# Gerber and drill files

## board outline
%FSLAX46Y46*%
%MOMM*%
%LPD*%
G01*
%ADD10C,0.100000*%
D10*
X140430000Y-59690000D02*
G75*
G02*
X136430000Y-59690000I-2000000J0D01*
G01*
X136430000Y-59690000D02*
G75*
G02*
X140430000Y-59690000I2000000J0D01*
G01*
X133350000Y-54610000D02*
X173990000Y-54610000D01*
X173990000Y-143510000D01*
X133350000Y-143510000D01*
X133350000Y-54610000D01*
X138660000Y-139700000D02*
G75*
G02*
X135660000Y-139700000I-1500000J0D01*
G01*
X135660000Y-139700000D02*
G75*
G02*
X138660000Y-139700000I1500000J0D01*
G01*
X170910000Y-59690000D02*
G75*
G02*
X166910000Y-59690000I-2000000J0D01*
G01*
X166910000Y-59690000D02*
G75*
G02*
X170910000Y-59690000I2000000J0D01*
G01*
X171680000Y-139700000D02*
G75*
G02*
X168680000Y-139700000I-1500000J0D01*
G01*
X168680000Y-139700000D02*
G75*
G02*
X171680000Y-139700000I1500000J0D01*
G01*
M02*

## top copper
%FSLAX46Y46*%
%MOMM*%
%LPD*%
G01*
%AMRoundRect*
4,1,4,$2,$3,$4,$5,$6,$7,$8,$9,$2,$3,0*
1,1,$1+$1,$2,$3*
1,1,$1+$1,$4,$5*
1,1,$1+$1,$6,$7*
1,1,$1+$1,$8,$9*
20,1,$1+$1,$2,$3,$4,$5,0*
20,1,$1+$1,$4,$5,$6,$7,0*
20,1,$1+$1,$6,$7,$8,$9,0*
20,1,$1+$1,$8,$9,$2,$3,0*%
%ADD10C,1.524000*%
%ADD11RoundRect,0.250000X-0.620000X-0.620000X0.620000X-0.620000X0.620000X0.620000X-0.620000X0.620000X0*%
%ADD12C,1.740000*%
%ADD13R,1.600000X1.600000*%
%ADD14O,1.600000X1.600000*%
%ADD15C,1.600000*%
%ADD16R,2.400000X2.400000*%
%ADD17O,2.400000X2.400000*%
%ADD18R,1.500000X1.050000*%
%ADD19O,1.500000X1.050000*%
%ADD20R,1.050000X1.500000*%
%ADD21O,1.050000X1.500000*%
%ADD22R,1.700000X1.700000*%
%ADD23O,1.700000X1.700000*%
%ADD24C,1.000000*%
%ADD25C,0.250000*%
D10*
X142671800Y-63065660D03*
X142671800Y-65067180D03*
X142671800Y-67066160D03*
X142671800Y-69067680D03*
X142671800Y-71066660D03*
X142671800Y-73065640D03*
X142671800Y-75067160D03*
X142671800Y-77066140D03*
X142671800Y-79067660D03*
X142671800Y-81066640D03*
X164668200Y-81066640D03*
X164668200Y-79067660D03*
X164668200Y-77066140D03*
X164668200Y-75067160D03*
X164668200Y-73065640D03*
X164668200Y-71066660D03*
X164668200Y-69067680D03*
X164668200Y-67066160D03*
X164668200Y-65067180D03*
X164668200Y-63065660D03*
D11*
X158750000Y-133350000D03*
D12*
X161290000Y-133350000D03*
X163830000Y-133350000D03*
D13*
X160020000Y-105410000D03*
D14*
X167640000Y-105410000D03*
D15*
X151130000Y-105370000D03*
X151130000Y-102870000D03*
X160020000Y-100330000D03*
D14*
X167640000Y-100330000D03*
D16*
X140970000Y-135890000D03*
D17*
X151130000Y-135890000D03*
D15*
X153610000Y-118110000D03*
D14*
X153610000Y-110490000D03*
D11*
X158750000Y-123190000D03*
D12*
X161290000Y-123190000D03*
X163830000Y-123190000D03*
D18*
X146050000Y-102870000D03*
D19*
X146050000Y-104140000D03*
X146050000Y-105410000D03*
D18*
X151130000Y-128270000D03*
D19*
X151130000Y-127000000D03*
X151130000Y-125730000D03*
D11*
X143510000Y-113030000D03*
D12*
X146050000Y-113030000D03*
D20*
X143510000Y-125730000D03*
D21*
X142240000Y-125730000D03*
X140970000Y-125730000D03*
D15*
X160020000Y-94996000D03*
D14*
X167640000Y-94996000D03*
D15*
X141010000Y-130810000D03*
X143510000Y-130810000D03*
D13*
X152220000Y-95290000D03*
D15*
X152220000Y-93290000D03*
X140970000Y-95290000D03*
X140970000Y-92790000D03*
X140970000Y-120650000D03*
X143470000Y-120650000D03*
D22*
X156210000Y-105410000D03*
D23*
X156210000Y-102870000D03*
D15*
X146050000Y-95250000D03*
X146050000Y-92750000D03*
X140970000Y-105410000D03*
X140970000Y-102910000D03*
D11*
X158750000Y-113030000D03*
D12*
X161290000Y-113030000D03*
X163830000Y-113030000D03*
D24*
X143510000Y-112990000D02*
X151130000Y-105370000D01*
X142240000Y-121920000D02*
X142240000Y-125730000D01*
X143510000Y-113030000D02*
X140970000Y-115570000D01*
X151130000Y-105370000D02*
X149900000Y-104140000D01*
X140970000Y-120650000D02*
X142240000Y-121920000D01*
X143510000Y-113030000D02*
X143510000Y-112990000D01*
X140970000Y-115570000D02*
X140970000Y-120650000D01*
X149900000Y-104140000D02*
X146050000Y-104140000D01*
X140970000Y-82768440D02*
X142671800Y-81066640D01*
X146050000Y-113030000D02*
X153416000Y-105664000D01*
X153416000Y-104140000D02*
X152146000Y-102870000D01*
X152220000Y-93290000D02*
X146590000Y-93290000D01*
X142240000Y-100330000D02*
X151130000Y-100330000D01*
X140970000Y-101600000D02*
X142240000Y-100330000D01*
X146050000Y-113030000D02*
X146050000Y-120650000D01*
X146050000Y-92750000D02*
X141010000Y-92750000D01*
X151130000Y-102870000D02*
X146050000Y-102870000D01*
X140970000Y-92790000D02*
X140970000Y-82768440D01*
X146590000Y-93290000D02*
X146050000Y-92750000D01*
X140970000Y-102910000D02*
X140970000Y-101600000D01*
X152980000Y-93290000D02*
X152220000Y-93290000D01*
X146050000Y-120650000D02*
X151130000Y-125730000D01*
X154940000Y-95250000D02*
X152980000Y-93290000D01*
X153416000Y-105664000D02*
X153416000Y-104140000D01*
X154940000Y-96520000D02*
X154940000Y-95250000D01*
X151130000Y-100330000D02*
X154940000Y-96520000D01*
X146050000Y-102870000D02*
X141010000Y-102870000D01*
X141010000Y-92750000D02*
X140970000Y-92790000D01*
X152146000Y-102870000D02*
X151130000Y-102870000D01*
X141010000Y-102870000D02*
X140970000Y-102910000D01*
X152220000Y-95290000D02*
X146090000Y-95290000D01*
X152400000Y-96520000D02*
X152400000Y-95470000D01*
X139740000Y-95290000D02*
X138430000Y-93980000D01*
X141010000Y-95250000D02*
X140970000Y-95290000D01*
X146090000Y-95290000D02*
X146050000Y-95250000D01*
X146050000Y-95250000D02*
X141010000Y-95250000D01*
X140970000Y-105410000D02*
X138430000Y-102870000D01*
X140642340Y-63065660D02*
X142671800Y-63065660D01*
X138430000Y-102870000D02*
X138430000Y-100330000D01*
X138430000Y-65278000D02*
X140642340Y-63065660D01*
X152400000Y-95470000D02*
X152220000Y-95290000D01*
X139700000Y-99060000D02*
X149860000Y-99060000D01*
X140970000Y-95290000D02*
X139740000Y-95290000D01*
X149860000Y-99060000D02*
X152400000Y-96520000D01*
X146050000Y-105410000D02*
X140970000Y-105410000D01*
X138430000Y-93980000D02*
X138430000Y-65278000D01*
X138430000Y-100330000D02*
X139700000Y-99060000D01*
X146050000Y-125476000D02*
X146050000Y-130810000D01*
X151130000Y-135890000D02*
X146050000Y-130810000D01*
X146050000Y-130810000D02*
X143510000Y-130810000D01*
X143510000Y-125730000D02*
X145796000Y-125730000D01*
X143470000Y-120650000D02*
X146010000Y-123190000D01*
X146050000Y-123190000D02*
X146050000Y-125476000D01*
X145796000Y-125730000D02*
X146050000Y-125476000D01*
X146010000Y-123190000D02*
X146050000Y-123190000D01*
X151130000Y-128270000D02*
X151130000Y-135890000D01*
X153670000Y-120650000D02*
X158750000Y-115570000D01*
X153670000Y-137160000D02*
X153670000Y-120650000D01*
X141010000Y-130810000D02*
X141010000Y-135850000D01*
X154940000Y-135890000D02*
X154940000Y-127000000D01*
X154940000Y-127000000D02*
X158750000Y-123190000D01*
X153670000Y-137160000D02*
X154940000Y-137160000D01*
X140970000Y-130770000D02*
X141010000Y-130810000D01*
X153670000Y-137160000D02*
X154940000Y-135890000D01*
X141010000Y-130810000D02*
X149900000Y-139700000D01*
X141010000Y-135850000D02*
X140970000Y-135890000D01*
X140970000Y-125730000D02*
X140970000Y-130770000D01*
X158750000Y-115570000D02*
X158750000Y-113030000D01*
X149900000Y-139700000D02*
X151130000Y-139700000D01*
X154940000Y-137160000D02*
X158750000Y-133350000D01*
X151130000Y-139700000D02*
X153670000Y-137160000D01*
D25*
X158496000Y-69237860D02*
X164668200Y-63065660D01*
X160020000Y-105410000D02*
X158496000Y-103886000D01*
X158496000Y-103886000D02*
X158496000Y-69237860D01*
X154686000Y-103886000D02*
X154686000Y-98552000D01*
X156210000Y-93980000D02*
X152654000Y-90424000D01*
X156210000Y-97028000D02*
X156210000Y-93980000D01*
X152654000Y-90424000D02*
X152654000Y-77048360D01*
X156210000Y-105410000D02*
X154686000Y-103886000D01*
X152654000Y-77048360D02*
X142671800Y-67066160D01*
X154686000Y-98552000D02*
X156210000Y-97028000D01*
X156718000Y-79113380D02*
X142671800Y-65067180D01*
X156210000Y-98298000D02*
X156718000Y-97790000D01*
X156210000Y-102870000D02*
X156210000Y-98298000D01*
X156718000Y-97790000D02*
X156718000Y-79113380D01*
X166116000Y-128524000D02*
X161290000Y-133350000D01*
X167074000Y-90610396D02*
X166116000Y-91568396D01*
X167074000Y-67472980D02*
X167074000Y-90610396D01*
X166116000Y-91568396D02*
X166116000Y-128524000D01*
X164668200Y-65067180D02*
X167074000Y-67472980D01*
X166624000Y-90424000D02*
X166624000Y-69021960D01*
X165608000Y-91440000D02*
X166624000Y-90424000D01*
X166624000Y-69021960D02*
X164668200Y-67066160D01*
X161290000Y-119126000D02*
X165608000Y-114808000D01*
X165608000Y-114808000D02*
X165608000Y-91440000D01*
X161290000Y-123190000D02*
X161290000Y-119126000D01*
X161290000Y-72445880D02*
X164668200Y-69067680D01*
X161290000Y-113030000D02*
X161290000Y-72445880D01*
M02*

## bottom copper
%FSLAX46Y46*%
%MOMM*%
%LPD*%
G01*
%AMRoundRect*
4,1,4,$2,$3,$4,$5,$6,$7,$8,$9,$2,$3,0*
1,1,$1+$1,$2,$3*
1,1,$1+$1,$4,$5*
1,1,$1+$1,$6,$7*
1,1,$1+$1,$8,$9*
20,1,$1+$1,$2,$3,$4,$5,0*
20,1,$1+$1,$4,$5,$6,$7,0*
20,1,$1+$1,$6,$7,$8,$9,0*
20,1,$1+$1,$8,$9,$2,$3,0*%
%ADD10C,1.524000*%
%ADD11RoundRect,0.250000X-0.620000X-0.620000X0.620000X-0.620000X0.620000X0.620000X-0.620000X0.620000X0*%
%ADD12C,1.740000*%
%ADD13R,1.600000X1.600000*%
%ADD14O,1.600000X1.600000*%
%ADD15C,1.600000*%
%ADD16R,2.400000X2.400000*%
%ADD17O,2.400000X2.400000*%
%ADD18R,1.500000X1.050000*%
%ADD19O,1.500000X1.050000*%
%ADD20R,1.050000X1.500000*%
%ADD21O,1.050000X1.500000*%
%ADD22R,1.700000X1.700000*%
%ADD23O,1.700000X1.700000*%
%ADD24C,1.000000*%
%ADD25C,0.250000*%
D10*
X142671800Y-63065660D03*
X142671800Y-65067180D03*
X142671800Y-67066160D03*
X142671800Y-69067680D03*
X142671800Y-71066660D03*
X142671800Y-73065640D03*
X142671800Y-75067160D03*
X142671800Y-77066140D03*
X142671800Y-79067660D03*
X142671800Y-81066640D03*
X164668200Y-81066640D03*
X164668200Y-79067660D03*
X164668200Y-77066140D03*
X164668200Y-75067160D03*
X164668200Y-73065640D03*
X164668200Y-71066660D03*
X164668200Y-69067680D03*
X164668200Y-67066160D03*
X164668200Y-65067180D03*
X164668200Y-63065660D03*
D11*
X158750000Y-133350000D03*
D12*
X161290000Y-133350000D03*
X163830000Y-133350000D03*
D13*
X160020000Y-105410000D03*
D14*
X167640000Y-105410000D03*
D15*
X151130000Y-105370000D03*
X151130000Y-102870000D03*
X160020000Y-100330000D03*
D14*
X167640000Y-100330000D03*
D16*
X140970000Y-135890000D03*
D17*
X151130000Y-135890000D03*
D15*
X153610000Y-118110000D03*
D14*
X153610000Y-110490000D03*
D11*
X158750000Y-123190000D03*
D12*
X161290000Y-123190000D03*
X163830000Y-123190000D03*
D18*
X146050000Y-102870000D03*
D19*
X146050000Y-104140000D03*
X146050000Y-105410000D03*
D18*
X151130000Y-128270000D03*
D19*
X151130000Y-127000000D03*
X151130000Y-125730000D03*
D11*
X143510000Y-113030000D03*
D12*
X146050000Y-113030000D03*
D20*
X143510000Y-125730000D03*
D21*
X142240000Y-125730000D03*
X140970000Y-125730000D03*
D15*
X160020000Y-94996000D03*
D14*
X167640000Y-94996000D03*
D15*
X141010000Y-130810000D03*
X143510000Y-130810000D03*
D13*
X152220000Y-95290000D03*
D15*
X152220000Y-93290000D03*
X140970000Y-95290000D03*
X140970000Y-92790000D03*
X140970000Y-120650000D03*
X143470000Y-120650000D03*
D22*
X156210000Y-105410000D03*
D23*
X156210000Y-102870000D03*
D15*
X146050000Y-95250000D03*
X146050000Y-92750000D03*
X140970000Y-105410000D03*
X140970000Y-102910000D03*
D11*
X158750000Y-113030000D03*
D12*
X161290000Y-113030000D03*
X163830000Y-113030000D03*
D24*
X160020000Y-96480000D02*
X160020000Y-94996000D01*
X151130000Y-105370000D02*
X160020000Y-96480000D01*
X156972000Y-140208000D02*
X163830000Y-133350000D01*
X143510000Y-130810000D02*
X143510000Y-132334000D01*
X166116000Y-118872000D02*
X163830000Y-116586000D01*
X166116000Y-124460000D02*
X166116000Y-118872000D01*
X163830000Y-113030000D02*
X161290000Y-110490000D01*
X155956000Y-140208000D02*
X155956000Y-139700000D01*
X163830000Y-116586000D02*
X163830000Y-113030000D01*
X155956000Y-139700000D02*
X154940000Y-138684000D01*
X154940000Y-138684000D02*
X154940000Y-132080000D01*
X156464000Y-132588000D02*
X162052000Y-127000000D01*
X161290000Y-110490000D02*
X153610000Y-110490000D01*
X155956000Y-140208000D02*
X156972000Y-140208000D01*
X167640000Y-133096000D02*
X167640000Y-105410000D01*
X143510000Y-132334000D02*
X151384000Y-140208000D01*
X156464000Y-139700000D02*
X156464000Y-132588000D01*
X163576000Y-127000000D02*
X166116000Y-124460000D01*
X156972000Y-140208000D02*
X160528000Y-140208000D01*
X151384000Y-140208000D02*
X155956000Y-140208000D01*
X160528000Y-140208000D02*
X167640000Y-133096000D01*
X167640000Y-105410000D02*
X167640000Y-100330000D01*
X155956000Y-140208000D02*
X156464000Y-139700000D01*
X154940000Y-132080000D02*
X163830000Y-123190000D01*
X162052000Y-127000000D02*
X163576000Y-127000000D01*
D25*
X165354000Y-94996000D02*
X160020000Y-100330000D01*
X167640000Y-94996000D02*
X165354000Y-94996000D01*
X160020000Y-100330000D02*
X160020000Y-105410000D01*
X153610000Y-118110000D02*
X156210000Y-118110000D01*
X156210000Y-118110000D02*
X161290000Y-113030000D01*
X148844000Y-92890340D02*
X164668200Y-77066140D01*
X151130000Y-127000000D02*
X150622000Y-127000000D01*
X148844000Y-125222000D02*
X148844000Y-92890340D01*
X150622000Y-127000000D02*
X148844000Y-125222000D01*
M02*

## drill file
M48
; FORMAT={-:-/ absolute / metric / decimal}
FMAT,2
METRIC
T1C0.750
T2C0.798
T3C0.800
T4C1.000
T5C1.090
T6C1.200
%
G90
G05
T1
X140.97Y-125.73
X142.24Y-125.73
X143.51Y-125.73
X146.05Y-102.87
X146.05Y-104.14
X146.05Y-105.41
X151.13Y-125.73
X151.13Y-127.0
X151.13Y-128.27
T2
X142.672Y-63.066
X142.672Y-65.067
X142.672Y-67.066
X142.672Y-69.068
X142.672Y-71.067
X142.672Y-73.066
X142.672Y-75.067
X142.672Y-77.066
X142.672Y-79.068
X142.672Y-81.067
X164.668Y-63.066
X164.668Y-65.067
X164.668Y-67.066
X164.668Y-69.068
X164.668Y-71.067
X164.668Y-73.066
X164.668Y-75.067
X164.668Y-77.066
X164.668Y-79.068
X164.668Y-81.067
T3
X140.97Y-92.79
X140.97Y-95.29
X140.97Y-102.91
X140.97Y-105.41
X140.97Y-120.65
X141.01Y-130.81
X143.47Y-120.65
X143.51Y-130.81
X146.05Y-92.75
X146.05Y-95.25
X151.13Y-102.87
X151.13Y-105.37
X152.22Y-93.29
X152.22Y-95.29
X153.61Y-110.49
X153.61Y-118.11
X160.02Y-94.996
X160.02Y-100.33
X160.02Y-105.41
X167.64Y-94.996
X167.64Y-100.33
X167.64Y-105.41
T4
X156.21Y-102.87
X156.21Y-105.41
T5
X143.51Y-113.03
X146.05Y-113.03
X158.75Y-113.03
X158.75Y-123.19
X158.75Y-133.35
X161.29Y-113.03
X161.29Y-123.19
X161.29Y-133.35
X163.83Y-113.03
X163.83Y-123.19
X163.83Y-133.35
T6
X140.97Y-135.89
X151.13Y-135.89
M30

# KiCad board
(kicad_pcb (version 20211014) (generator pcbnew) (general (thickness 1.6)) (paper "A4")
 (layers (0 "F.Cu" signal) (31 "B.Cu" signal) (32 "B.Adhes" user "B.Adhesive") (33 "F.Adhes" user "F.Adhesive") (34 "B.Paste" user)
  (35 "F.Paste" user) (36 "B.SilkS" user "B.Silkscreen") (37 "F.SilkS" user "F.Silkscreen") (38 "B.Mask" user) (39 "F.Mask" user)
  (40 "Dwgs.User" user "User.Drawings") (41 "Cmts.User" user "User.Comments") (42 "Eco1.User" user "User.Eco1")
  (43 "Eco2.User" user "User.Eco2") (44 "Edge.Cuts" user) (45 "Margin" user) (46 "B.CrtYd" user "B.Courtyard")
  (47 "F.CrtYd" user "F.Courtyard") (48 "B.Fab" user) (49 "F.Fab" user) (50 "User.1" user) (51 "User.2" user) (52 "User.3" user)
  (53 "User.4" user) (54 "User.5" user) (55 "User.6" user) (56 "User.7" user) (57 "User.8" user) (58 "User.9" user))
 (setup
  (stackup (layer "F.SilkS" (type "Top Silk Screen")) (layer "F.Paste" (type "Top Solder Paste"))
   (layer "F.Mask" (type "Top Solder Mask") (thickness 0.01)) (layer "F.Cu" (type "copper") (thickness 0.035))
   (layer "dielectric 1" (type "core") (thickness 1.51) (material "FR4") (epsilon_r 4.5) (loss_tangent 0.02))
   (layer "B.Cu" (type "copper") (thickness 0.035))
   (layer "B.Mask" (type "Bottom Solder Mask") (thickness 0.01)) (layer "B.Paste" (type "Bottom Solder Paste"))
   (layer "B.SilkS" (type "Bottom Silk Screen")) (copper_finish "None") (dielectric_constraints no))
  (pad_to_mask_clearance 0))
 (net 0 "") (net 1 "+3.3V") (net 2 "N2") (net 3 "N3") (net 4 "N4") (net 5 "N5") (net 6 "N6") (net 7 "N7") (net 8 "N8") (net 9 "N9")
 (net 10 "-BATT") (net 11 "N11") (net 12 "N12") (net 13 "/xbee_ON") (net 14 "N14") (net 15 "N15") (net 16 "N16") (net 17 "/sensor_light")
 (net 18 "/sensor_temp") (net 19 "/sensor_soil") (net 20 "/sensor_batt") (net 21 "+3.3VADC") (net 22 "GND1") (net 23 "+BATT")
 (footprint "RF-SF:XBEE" (layer "F.Cu") (at 153.67 83.06562)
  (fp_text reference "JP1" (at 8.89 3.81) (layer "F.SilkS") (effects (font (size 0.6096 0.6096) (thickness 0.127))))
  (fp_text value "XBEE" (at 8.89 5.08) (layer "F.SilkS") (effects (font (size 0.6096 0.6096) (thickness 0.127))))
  (pad "1" thru_hole circle locked (at -10.9982 -19.99996) (size 1.524 1.524) (drill 0.79756) (layers *.Cu *.Mask) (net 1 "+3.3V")
   (solder_mask_margin 0.1016))
  (pad "2" thru_hole circle locked (at -10.9982 -17.99844) (size 1.524 1.524) (drill 0.79756) (layers *.Cu *.Mask) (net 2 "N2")
   (solder_mask_margin 0.1016))
  (pad "3" thru_hole circle locked (at -10.9982 -15.99946) (size 1.524 1.524) (drill 0.79756) (layers *.Cu *.Mask) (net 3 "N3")
   (solder_mask_margin 0.1016))
  (pad "4" thru_hole circle locked (at -10.9982 -13.99794) (size 1.524 1.524) (drill 0.79756) (layers *.Cu *.Mask) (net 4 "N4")
   (solder_mask_margin 0.1016))
  (pad "5" thru_hole circle locked (at -10.9982 -11.99896) (size 1.524 1.524) (drill 0.79756) (layers *.Cu *.Mask) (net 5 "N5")
   (solder_mask_margin 0.1016))
  (pad "6" thru_hole circle locked (at -10.9982 -9.99998) (size 1.524 1.524) (drill 0.79756) (layers *.Cu *.Mask) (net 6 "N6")
   (solder_mask_margin 0.1016))
  (pad "7" thru_hole circle locked (at -10.9982 -7.99846) (size 1.524 1.524) (drill 0.79756) (layers *.Cu *.Mask) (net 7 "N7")
   (solder_mask_margin 0.1016))
  (pad "8" thru_hole circle locked (at -10.9982 -5.99948) (size 1.524 1.524) (drill 0.79756) (layers *.Cu *.Mask) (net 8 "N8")
   (solder_mask_margin 0.1016))
  (pad "9" thru_hole circle locked (at -10.9982 -3.99796) (size 1.524 1.524) (drill 0.79756) (layers *.Cu *.Mask) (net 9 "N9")
   (solder_mask_margin 0.1016))
  (pad "10" thru_hole circle locked (at -10.9982 -1.99898) (size 1.524 1.524) (drill 0.79756) (layers *.Cu *.Mask) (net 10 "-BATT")
   (solder_mask_margin 0.1016))
  (pad "11" thru_hole circle locked (at 10.9982 -1.99898) (size 1.524 1.524) (drill 0.79756) (layers *.Cu *.Mask) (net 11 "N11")
   (solder_mask_margin 0.1016))
  (pad "12" thru_hole circle locked (at 10.9982 -3.99796) (size 1.524 1.524) (drill 0.79756) (layers *.Cu *.Mask) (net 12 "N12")
   (solder_mask_margin 0.1016))
  (pad "13" thru_hole circle locked (at 10.9982 -5.99948) (size 1.524 1.524) (drill 0.79756) (layers *.Cu *.Mask) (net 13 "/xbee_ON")
   (solder_mask_margin 0.1016))
  (pad "14" thru_hole circle locked (at 10.9982 -7.99846) (size 1.524 1.524) (drill 0.79756) (layers *.Cu *.Mask) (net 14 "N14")
   (solder_mask_margin 0.1016))
  (pad "15" thru_hole circle locked (at 10.9982 -9.99998) (size 1.524 1.524) (drill 0.79756) (layers *.Cu *.Mask) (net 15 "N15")
   (solder_mask_margin 0.1016))
  (pad "16" thru_hole circle locked (at 10.9982 -11.99896) (size 1.524 1.524) (drill 0.79756) (layers *.Cu *.Mask) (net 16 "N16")
   (solder_mask_margin 0.1016))
  (pad "17" thru_hole circle locked (at 10.9982 -13.99794) (size 1.524 1.524) (drill 0.79756) (layers *.Cu *.Mask) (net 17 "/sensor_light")
   (solder_mask_margin 0.1016))
  (pad "18" thru_hole circle locked (at 10.9982 -15.99946) (size 1.524 1.524) (drill 0.79756) (layers *.Cu *.Mask) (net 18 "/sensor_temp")
   (solder_mask_margin 0.1016))
  (pad "19" thru_hole circle locked (at 10.9982 -17.99844) (size 1.524 1.524) (drill 0.79756) (layers *.Cu *.Mask) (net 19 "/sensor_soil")
   (solder_mask_margin 0.1016))
  (pad "20" thru_hole circle locked (at 10.9982 -19.99996) (size 1.524 1.524) (drill 0.79756) (layers *.Cu *.Mask) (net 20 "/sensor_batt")
   (solder_mask_margin 0.1016)))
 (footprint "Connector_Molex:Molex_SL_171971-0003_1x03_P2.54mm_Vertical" (layer "F.Cu") (at 158.75 133.35)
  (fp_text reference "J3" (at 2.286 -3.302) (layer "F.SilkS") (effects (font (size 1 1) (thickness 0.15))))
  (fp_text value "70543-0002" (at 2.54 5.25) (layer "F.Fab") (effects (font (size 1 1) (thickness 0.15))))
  (pad "1" thru_hole roundrect (at 0 0) (size 1.74 1.74) (drill 1.09) (layers *.Cu *.Mask) (roundrect_rratio 0.1436781609)
   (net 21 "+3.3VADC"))
  (pad "2" thru_hole circle (at 2.54 0) (size 1.74 1.74) (drill 1.09) (layers *.Cu *.Mask) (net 19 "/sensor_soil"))
  (pad "3" thru_hole circle (at 5.08 0) (size 1.74 1.74) (drill 1.09) (layers *.Cu *.Mask) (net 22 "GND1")))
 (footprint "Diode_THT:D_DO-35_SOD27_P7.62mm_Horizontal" (layer "F.Cu") (at 160.02 105.41)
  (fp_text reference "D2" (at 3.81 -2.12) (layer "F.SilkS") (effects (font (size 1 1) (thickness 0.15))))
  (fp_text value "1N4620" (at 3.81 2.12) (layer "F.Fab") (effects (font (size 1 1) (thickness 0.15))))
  (pad "1" thru_hole rect (at 0 0) (size 1.6 1.6) (drill 0.8) (layers *.Cu *.Mask) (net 20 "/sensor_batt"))
  (pad "2" thru_hole oval (at 7.62 0) (size 1.6 1.6) (drill 0.8) (layers *.Cu *.Mask) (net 22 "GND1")))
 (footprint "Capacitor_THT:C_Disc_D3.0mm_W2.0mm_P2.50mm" (layer "F.Cu") (at 151.13 105.37 90)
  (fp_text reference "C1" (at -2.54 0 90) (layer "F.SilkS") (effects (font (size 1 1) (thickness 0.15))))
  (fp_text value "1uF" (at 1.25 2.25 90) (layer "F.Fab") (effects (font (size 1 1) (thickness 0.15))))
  (pad "1" thru_hole circle (at 0 0 90) (size 1.6 1.6) (drill 0.8) (layers *.Cu *.Mask) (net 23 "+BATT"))
  (pad "2" thru_hole circle (at 2.5 0 90) (size 1.6 1.6) (drill 0.8) (layers *.Cu *.Mask) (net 10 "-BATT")))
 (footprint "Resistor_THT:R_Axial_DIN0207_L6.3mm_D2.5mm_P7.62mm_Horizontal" (layer "F.Cu") (at 160.02 100.33)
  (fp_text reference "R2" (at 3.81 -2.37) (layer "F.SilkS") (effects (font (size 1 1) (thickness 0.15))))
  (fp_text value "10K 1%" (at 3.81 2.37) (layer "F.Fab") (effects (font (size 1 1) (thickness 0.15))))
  (pad "1" thru_hole circle (at 0 0) (size 1.6 1.6) (drill 0.8) (layers *.Cu *.Mask) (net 20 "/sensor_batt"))
  (pad "2" thru_hole oval (at 7.62 0) (size 1.6 1.6) (drill 0.8) (layers *.Cu *.Mask) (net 22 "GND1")))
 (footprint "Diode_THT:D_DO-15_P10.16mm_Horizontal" (layer "F.Cu") (at 140.97 135.89)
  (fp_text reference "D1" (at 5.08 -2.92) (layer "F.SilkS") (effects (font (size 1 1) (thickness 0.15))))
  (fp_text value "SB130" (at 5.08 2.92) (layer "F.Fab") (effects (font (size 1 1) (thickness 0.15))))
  (pad "1" thru_hole rect (at 0 0) (size 2.4 2.4) (drill 1.2) (layers *.Cu *.Mask) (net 21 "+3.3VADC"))
  (pad "2" thru_hole oval (at 10.16 0) (size 2.4 2.4) (drill 1.2) (layers *.Cu *.Mask) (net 22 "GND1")))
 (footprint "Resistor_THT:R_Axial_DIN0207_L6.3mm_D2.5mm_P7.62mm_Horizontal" (layer "F.Cu") (at 153.61 118.11 90)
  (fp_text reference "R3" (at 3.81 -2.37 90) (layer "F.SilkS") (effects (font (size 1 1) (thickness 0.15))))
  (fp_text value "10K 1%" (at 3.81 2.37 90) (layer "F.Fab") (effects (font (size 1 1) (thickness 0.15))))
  (pad "1" thru_hole circle (at 0 0 90) (size 1.6 1.6) (drill 0.8) (layers *.Cu *.Mask) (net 17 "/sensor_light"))
  (pad "2" thru_hole oval (at 7.62 0 90) (size 1.6 1.6) (drill 0.8) (layers *.Cu *.Mask) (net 22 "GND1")))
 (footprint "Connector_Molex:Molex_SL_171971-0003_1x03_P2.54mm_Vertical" (layer "F.Cu") (at 158.75 123.19)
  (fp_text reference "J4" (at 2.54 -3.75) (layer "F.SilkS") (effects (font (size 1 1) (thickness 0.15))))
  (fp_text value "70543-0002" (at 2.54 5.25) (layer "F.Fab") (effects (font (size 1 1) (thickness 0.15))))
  (pad "1" thru_hole roundrect (at 0 0) (size 1.74 1.74) (drill 1.09) (layers *.Cu *.Mask) (roundrect_rratio 0.1436781609)
   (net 21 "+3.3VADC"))
  (pad "2" thru_hole circle (at 2.54 0) (size 1.74 1.74) (drill 1.09) (layers *.Cu *.Mask) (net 18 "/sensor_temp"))
  (pad "3" thru_hole circle (at 5.08 0) (size 1.74 1.74) (drill 1.09) (layers *.Cu *.Mask) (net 22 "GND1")))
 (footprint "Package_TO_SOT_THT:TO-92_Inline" (layer "F.Cu") (at 146.05 102.87 -90)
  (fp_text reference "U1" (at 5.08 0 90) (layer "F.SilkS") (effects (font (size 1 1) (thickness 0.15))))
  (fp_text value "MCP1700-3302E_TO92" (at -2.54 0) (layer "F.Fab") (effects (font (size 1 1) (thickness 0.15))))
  (pad "1" thru_hole rect (at 0 0 270) (size 1.05 1.5) (drill 0.75) (layers *.Cu *.Mask) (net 10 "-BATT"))
  (pad "2" thru_hole oval (at 1.27 0 270) (size 1.05 1.5) (drill 0.75) (layers *.Cu *.Mask) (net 23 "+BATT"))
  (pad "3" thru_hole oval (at 2.54 0 270) (size 1.05 1.5) (drill 0.75) (layers *.Cu *.Mask) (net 1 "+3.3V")))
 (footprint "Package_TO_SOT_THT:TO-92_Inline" (layer "F.Cu") (at 151.13 128.27 90)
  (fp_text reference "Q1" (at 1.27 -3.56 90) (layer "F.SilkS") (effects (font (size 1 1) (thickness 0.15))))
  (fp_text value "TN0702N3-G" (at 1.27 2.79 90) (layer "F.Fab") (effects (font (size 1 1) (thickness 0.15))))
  (pad "1" thru_hole rect (at 0 0 90) (size 1.05 1.5) (drill 0.75) (layers *.Cu *.Mask) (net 22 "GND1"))
  (pad "2" thru_hole oval (at 1.27 0 90) (size 1.05 1.5) (drill 0.75) (layers *.Cu *.Mask) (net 13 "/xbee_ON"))
  (pad "3" thru_hole oval (at 2.54 0 90) (size 1.05 1.5) (drill 0.75) (layers *.Cu *.Mask) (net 10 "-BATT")))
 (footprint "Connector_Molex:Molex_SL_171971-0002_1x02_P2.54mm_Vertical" (layer "F.Cu") (at 143.51 113.03)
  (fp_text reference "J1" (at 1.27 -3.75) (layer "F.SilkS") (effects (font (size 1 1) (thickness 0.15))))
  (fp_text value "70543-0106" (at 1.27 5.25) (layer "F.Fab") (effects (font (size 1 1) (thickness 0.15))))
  (pad "1" thru_hole roundrect (at 0 0) (size 1.74 1.74) (drill 1.09) (layers *.Cu *.Mask) (roundrect_rratio 0.1436781609) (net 23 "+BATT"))
  (pad "2" thru_hole circle (at 2.54 0) (size 1.74 1.74) (drill 1.09) (layers *.Cu *.Mask) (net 10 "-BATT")))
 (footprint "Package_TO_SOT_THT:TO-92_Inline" (layer "F.Cu") (at 143.51 125.73 180)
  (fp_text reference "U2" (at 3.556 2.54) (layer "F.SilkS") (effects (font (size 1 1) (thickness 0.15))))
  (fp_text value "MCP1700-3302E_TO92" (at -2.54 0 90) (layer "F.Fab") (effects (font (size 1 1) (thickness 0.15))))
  (pad "1" thru_hole rect (at 0 0 180) (size 1.05 1.5) (drill 0.75) (layers *.Cu *.Mask) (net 22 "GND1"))
  (pad "2" thru_hole oval (at 1.27 0 180) (size 1.05 1.5) (drill 0.75) (layers *.Cu *.Mask) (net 23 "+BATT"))
  (pad "3" thru_hole oval (at 2.54 0 180) (size 1.05 1.5) (drill 0.75) (layers *.Cu *.Mask) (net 21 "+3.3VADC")))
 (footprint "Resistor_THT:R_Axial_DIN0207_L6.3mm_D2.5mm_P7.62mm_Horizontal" (layer "F.Cu") (at 160.02 94.996)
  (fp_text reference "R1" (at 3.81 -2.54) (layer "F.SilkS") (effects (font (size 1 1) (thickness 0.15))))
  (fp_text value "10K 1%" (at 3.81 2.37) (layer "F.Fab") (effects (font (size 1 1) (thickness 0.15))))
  (pad "1" thru_hole circle (at 0 0) (size 1.6 1.6) (drill 0.8) (layers *.Cu *.Mask) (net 23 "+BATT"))
  (pad "2" thru_hole oval (at 7.62 0) (size 1.6 1.6) (drill 0.8) (layers *.Cu *.Mask) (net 20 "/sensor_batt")))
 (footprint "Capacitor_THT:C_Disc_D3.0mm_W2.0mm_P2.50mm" (layer "F.Cu") (at 141.01 130.81)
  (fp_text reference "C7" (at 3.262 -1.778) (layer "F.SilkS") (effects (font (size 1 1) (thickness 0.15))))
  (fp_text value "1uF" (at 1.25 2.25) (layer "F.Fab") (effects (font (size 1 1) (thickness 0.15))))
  (pad "1" thru_hole circle (at 0 0) (size 1.6 1.6) (drill 0.8) (layers *.Cu *.Mask) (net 21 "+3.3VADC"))
  (pad "2" thru_hole circle (at 2.5 0) (size 1.6 1.6) (drill 0.8) (layers *.Cu *.Mask) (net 22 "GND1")))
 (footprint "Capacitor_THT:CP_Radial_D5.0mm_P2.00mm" (layer "F.Cu") (at 152.22 95.29 90)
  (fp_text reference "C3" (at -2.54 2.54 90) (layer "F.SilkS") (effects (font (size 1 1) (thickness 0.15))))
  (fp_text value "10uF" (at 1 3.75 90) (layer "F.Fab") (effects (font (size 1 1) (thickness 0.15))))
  (pad "1" thru_hole rect (at 0 0 90) (size 1.6 1.6) (drill 0.8) (layers *.Cu *.Mask) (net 1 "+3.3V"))
  (pad "2" thru_hole circle (at 2 0 90) (size 1.6 1.6) (drill 0.8) (layers *.Cu *.Mask) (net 10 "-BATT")))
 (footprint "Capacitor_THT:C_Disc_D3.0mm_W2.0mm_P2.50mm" (layer "F.Cu") (at 140.97 95.29 90)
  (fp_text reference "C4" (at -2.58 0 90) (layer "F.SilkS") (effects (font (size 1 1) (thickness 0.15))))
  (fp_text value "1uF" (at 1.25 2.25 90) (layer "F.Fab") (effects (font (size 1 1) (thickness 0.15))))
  (pad "1" thru_hole circle (at 0 0 90) (size 1.6 1.6) (drill 0.8) (layers *.Cu *.Mask) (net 1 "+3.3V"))
  (pad "2" thru_hole circle (at 2.5 0 90) (size 1.6 1.6) (drill 0.8) (layers *.Cu *.Mask) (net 10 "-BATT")))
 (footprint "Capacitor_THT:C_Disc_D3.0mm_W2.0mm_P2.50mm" (layer "F.Cu") (at 140.97 120.65)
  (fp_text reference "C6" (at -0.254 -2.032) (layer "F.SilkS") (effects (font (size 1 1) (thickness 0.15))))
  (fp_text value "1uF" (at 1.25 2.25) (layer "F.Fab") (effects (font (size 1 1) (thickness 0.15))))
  (pad "1" thru_hole circle (at 0 0) (size 1.6 1.6) (drill 0.8) (layers *.Cu *.Mask) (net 23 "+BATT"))
  (pad "2" thru_hole circle (at 2.5 0) (size 1.6 1.6) (drill 0.8) (layers *.Cu *.Mask) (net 22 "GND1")))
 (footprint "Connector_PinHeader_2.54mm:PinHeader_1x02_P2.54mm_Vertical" (layer "F.Cu") (at 156.21 105.41 180)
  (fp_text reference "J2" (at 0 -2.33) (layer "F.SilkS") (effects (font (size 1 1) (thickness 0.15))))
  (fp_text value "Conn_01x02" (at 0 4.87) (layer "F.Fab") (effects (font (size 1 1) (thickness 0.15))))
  (pad "1" thru_hole rect (at 0 0 180) (size 1.7 1.7) (drill 1) (layers *.Cu *.Mask) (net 3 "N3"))
  (pad "2" thru_hole oval (at 0 2.54 180) (size 1.7 1.7) (drill 1) (layers *.Cu *.Mask) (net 2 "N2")))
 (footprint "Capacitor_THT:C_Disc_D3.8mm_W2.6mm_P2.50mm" (layer "F.Cu") (at 146.05 95.25 90)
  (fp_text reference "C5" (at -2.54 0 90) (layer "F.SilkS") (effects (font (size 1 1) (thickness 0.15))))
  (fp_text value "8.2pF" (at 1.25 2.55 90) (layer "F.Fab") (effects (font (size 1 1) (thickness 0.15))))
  (pad "1" thru_hole circle (at 0 0 90) (size 1.6 1.6) (drill 0.8) (layers *.Cu *.Mask) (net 1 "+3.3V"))
  (pad "2" thru_hole circle (at 2.5 0 90) (size 1.6 1.6) (drill 0.8) (layers *.Cu *.Mask) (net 10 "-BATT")))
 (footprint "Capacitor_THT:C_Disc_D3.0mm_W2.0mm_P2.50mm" (layer "F.Cu") (at 140.97 105.41 90)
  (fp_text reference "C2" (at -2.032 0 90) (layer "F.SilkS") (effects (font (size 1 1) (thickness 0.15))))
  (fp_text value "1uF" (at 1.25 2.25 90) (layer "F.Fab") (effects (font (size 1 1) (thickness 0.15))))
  (pad "1" thru_hole circle (at 0 0 90) (size 1.6 1.6) (drill 0.8) (layers *.Cu *.Mask) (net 1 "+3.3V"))
  (pad "2" thru_hole circle (at 2.5 0 90) (size 1.6 1.6) (drill 0.8) (layers *.Cu *.Mask) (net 10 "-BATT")))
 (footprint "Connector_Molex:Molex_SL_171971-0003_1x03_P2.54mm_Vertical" (layer "F.Cu") (at 158.75 113.03)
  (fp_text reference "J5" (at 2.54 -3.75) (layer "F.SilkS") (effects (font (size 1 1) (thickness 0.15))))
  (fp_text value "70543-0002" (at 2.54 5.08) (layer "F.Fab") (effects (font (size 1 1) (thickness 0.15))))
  (pad "1" thru_hole roundrect (at 0 0) (size 1.74 1.74) (drill 1.09) (layers *.Cu *.Mask) (roundrect_rratio 0.1436781609)
   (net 21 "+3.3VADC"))
  (pad "2" thru_hole circle (at 2.54 0) (size 1.74 1.74) (drill 1.09) (layers *.Cu *.Mask) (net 17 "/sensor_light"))
  (pad "3" thru_hole circle (at 5.08 0) (size 1.74 1.74) (drill 1.09) (layers *.Cu *.Mask) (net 22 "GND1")))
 (gr_circle (center 138.43 59.69) (end 140.43 59.69) (layer "Edge.Cuts") (width 0.1) (fill none))
 (gr_rect (start 133.35 143.51) (end 173.99 54.61) (layer "Edge.Cuts") (width 0.1) (fill none))
 (gr_circle (center 137.16 139.7) (end 138.66 139.7) (layer "Edge.Cuts") (width 0.1) (fill none))
 (gr_circle (center 168.91 59.69) (end 170.91 59.69) (layer "Edge.Cuts") (width 0.1) (fill none))
 (gr_circle (center 170.18 139.7) (end 171.68 139.7) (layer "Edge.Cuts") (width 0.1) (fill none))
 (segment (start 143.51 112.99) (end 151.13 105.37) (width 1) (layer "F.Cu") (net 23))
 (segment (start 142.24 121.92) (end 142.24 125.73) (width 1) (layer "F.Cu") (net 23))
 (segment (start 143.51 113.03) (end 140.97 115.57) (width 1) (layer "F.Cu") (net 23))
 (segment (start 151.13 105.37) (end 149.9 104.14) (width 1) (layer "F.Cu") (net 23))
 (segment (start 140.97 120.65) (end 142.24 121.92) (width 1) (layer "F.Cu") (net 23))
 (segment (start 143.51 113.03) (end 143.51 112.99) (width 1) (layer "F.Cu") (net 23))
 (segment (start 140.97 115.57) (end 140.97 120.65) (width 1) (layer "F.Cu") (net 23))
 (segment (start 149.9 104.14) (end 146.05 104.14) (width 1) (layer "F.Cu") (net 23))
 (segment (start 160.02 96.48) (end 160.02 94.996) (width 1) (layer "B.Cu") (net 23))
 (segment (start 151.13 105.37) (end 160.02 96.48) (width 1) (layer "B.Cu") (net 23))
 (segment (start 140.97 82.76844) (end 142.6718 81.06664) (width 1) (layer "F.Cu") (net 10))
 (segment (start 146.05 113.03) (end 153.416 105.664) (width 1) (layer "F.Cu") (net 10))
 (segment (start 153.416 104.14) (end 152.146 102.87) (width 1) (layer "F.Cu") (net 10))
 (segment (start 152.22 93.29) (end 146.59 93.29) (width 1) (layer "F.Cu") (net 10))
 (segment (start 142.24 100.33) (end 151.13 100.33) (width 1) (layer "F.Cu") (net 10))
 (segment (start 140.97 101.6) (end 142.24 100.33) (width 1) (layer "F.Cu") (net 10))
 (segment (start 146.05 113.03) (end 146.05 120.65) (width 1) (layer "F.Cu") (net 10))
 (segment (start 146.05 92.75) (end 141.01 92.75) (width 1) (layer "F.Cu") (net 10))
 (segment (start 151.13 102.87) (end 146.05 102.87) (width 1) (layer "F.Cu") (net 10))
 (segment (start 140.97 92.79) (end 140.97 82.76844) (width 1) (layer "F.Cu") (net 10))
 (segment (start 146.59 93.29) (end 146.05 92.75) (width 1) (layer "F.Cu") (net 10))
 (segment (start 140.97 102.91) (end 140.97 101.6) (width 1) (layer "F.Cu") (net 10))
 (segment (start 152.98 93.29) (end 152.22 93.29) (width 1) (layer "F.Cu") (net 10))
 (segment (start 146.05 120.65) (end 151.13 125.73) (width 1) (layer "F.Cu") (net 10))
 (segment (start 154.94 95.25) (end 152.98 93.29) (width 1) (layer "F.Cu") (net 10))
 (segment (start 153.416 105.664) (end 153.416 104.14) (width 1) (layer "F.Cu") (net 10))
 (segment (start 154.94 96.52) (end 154.94 95.25) (width 1) (layer "F.Cu") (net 10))
 (segment (start 151.13 100.33) (end 154.94 96.52) (width 1) (layer "F.Cu") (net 10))
 (segment (start 146.05 102.87) (end 141.01 102.87) (width 1) (layer "F.Cu") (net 10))
 (segment (start 141.01 92.75) (end 140.97 92.79) (width 1) (layer "F.Cu") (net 10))
 (segment (start 152.146 102.87) (end 151.13 102.87) (width 1) (layer "F.Cu") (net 10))
 (segment (start 141.01 102.87) (end 140.97 102.91) (width 1) (layer "F.Cu") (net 10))
 (segment (start 152.22 95.29) (end 146.09 95.29) (width 1) (layer "F.Cu") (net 1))
 (segment (start 152.4 96.52) (end 152.4 95.47) (width 1) (layer "F.Cu") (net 1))
 (segment (start 139.74 95.29) (end 138.43 93.98) (width 1) (layer "F.Cu") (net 1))
 (segment (start 141.01 95.25) (end 140.97 95.29) (width 1) (layer "F.Cu") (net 1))
 (segment (start 146.09 95.29) (end 146.05 95.25) (width 1) (layer "F.Cu") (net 1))
 (segment (start 146.05 95.25) (end 141.01 95.25) (width 1) (layer "F.Cu") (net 1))
 (segment (start 140.97 105.41) (end 138.43 102.87) (width 1) (layer "F.Cu") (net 1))
 (segment (start 140.64234 63.06566) (end 142.6718 63.06566) (width 1) (layer "F.Cu") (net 1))
 (segment (start 138.43 102.87) (end 138.43 100.33) (width 1) (layer "F.Cu") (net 1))
 (segment (start 138.43 65.278) (end 140.64234 63.06566) (width 1) (layer "F.Cu") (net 1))
 (segment (start 152.4 95.47) (end 152.22 95.29) (width 1) (layer "F.Cu") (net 1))
 (segment (start 139.7 99.06) (end 149.86 99.06) (width 1) (layer "F.Cu") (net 1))
 (segment (start 140.97 95.29) (end 139.74 95.29) (width 1) (layer "F.Cu") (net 1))
 (segment (start 149.86 99.06) (end 152.4 96.52) (width 1) (layer "F.Cu") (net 1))
 (segment (start 146.05 105.41) (end 140.97 105.41) (width 1) (layer "F.Cu") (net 1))
 (segment (start 138.43 93.98) (end 138.43 65.278) (width 1) (layer "F.Cu") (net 1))
 (segment (start 138.43 100.33) (end 139.7 99.06) (width 1) (layer "F.Cu") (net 1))
 (segment (start 146.05 125.476) (end 146.05 130.81) (width 1) (layer "F.Cu") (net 22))
 (segment (start 151.13 135.89) (end 146.05 130.81) (width 1) (layer "F.Cu") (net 22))
 (segment (start 146.05 130.81) (end 143.51 130.81) (width 1) (layer "F.Cu") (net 22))
 (segment (start 143.51 125.73) (end 145.796 125.73) (width 1) (layer "F.Cu") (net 22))
 (segment (start 143.47 120.65) (end 146.01 123.19) (width 1) (layer "F.Cu") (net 22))
 (segment (start 146.05 123.19) (end 146.05 125.476) (width 1) (layer "F.Cu") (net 22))
 (segment (start 145.796 125.73) (end 146.05 125.476) (width 1) (layer "F.Cu") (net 22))
 (segment (start 146.01 123.19) (end 146.05 123.19) (width 1) (layer "F.Cu") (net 22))
 (segment (start 151.13 128.27) (end 151.13 135.89) (width 1) (layer "F.Cu") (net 22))
 (segment (start 156.972 140.208) (end 163.83 133.35) (width 1) (layer "B.Cu") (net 22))
 (segment (start 143.51 130.81) (end 143.51 132.334) (width 1) (layer "B.Cu") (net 22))
 (segment (start 166.116 118.872) (end 163.83 116.586) (width 1) (layer "B.Cu") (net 22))
 (segment (start 166.116 124.46) (end 166.116 118.872) (width 1) (layer "B.Cu") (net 22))
 (segment (start 163.83 113.03) (end 161.29 110.49) (width 1) (layer "B.Cu") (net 22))
 (segment (start 155.956 140.208) (end 155.956 139.7) (width 1) (layer "B.Cu") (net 22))
 (segment (start 163.83 116.586) (end 163.83 113.03) (width 1) (layer "B.Cu") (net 22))
 (segment (start 155.956 139.7) (end 154.94 138.684) (width 1) (layer "B.Cu") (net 22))
 (segment (start 154.94 138.684) (end 154.94 132.08) (width 1) (layer "B.Cu") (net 22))
 (segment (start 156.464 132.588) (end 162.052 127) (width 1) (layer "B.Cu") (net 22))
 (segment (start 161.29 110.49) (end 153.61 110.49) (width 1) (layer "B.Cu") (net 22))
 (segment (start 155.956 140.208) (end 156.972 140.208) (width 1) (layer "B.Cu") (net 22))
 (segment (start 167.64 133.096) (end 167.64 105.41) (width 1) (layer "B.Cu") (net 22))
 (segment (start 143.51 132.334) (end 151.384 140.208) (width 1) (layer "B.Cu") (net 22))
 (segment (start 156.464 139.7) (end 156.464 132.588) (width 1) (layer "B.Cu") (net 22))
 (segment (start 163.576 127) (end 166.116 124.46) (width 1) (layer "B.Cu") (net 22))
 (segment (start 156.972 140.208) (end 160.528 140.208) (width 1) (layer "B.Cu") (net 22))
 (segment (start 151.384 140.208) (end 155.956 140.208) (width 1) (layer "B.Cu") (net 22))
 (segment (start 160.528 140.208) (end 167.64 133.096) (width 1) (layer "B.Cu") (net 22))
 (segment (start 167.64 105.41) (end 167.64 100.33) (width 1) (layer "B.Cu") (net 22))
 (segment (start 155.956 140.208) (end 156.464 139.7) (width 1) (layer "B.Cu") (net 22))
 (segment (start 154.94 132.08) (end 163.83 123.19) (width 1) (layer "B.Cu") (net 22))
 (segment (start 162.052 127) (end 163.576 127) (width 1) (layer "B.Cu") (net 22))
 (segment (start 153.67 120.65) (end 158.75 115.57) (width 1) (layer "F.Cu") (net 21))
 (segment (start 153.67 137.16) (end 153.67 120.65) (width 1) (layer "F.Cu") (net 21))
 (segment (start 141.01 130.81) (end 141.01 135.85) (width 1) (layer "F.Cu") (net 21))
 (segment (start 154.94 135.89) (end 154.94 127) (width 1) (layer "F.Cu") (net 21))
 (segment (start 154.94 127) (end 158.75 123.19) (width 1) (layer "F.Cu") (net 21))
 (segment (start 153.67 137.16) (end 154.94 137.16) (width 1) (layer "F.Cu") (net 21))
 (segment (start 140.97 130.77) (end 141.01 130.81) (width 1) (layer "F.Cu") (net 21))
 (segment (start 153.67 137.16) (end 154.94 135.89) (width 1) (layer "F.Cu") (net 21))
 (segment (start 141.01 130.81) (end 149.9 139.7) (width 1) (layer "F.Cu") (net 21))
 (segment (start 141.01 135.85) (end 140.97 135.89) (width 1) (layer "F.Cu") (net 21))
 (segment (start 140.97 125.73) (end 140.97 130.77) (width 1) (layer "F.Cu") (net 21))
 (segment (start 158.75 115.57) (end 158.75 113.03) (width 1) (layer "F.Cu") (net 21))
 (segment (start 149.9 139.7) (end 151.13 139.7) (width 1) (layer "F.Cu") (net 21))
 (segment (start 154.94 137.16) (end 158.75 133.35) (width 1) (layer "F.Cu") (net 21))
 (segment (start 151.13 139.7) (end 153.67 137.16) (width 1) (layer "F.Cu") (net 21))
 (segment (start 158.496 69.23786) (end 164.6682 63.06566) (width 0.25) (layer "F.Cu") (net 20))
 (segment (start 160.02 105.41) (end 158.496 103.886) (width 0.25) (layer "F.Cu") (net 20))
 (segment (start 158.496 103.886) (end 158.496 69.23786) (width 0.25) (layer "F.Cu") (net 20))
 (segment (start 165.354 94.996) (end 160.02 100.33) (width 0.25) (layer "B.Cu") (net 20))
 (segment (start 167.64 94.996) (end 165.354 94.996) (width 0.25) (layer "B.Cu") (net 20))
 (segment (start 160.02 100.33) (end 160.02 105.41) (width 0.25) (layer "B.Cu") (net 20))
 (segment (start 154.686 103.886) (end 154.686 98.552) (width 0.25) (layer "F.Cu") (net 3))
 (segment (start 156.21 93.98) (end 152.654 90.424) (width 0.25) (layer "F.Cu") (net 3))
 (segment (start 156.21 97.028) (end 156.21 93.98) (width 0.25) (layer "F.Cu") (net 3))
 (segment (start 152.654 90.424) (end 152.654 77.04836) (width 0.25) (layer "F.Cu") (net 3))
 (segment (start 156.21 105.41) (end 154.686 103.886) (width 0.25) (layer "F.Cu") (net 3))
 (segment (start 152.654 77.04836) (end 142.6718 67.06616) (width 0.25) (layer "F.Cu") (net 3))
 (segment (start 154.686 98.552) (end 156.21 97.028) (width 0.25) (layer "F.Cu") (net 3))
 (segment (start 156.718 79.11338) (end 142.6718 65.06718) (width 0.25) (layer "F.Cu") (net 2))
 (segment (start 156.21 98.298) (end 156.718 97.79) (width 0.25) (layer "F.Cu") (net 2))
 (segment (start 156.21 102.87) (end 156.21 98.298) (width 0.25) (layer "F.Cu") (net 2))
 (segment (start 156.718 97.79) (end 156.718 79.11338) (width 0.25) (layer "F.Cu") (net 2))
 (segment (start 166.116 128.524) (end 161.29 133.35) (width 0.25) (layer "F.Cu") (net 19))
 (segment (start 167.074 90.610396) (end 166.116 91.568396) (width 0.25) (layer "F.Cu") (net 19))
 (segment (start 167.074 67.47298) (end 167.074 90.610396) (width 0.25) (layer "F.Cu") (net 19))
 (segment (start 166.116 91.568396) (end 166.116 128.524) (width 0.25) (layer "F.Cu") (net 19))
 (segment (start 164.6682 65.06718) (end 167.074 67.47298) (width 0.25) (layer "F.Cu") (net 19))
 (segment (start 166.624 90.424) (end 166.624 69.02196) (width 0.25) (layer "F.Cu") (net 18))
 (segment (start 165.608 91.44) (end 166.624 90.424) (width 0.25) (layer "F.Cu") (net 18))
 (segment (start 166.624 69.02196) (end 164.6682 67.06616) (width 0.25) (layer "F.Cu") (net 18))
 (segment (start 161.29 119.126) (end 165.608 114.808) (width 0.25) (layer "F.Cu") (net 18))
 (segment (start 165.608 114.808) (end 165.608 91.44) (width 0.25) (layer "F.Cu") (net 18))
 (segment (start 161.29 123.19) (end 161.29 119.126) (width 0.25) (layer "F.Cu") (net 18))
 (segment (start 161.29 72.44588) (end 164.6682 69.06768) (width 0.25) (layer "F.Cu") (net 17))
 (segment (start 161.29 113.03) (end 161.29 72.44588) (width 0.25) (layer "F.Cu") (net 17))
 (segment (start 153.61 118.11) (end 156.21 118.11) (width 0.25) (layer "B.Cu") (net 17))
 (segment (start 156.21 118.11) (end 161.29 113.03) (width 0.25) (layer "B.Cu") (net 17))
 (segment (start 148.844 92.89034) (end 164.6682 77.06614) (width 0.25) (layer "B.Cu") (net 13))
 (segment (start 151.13 127) (end 150.622 127) (width 0.25) (layer "B.Cu") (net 13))
 (segment (start 148.844 125.222) (end 148.844 92.89034) (width 0.25) (layer "B.Cu") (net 13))
 (segment (start 150.622 127) (end 148.844 125.222) (width 0.25) (layer "B.Cu") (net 13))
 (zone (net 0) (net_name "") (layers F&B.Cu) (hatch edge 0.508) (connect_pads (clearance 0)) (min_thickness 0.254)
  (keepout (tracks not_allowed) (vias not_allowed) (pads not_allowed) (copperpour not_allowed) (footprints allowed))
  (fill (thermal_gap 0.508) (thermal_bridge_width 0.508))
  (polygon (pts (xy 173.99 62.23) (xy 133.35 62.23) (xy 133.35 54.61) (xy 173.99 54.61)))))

